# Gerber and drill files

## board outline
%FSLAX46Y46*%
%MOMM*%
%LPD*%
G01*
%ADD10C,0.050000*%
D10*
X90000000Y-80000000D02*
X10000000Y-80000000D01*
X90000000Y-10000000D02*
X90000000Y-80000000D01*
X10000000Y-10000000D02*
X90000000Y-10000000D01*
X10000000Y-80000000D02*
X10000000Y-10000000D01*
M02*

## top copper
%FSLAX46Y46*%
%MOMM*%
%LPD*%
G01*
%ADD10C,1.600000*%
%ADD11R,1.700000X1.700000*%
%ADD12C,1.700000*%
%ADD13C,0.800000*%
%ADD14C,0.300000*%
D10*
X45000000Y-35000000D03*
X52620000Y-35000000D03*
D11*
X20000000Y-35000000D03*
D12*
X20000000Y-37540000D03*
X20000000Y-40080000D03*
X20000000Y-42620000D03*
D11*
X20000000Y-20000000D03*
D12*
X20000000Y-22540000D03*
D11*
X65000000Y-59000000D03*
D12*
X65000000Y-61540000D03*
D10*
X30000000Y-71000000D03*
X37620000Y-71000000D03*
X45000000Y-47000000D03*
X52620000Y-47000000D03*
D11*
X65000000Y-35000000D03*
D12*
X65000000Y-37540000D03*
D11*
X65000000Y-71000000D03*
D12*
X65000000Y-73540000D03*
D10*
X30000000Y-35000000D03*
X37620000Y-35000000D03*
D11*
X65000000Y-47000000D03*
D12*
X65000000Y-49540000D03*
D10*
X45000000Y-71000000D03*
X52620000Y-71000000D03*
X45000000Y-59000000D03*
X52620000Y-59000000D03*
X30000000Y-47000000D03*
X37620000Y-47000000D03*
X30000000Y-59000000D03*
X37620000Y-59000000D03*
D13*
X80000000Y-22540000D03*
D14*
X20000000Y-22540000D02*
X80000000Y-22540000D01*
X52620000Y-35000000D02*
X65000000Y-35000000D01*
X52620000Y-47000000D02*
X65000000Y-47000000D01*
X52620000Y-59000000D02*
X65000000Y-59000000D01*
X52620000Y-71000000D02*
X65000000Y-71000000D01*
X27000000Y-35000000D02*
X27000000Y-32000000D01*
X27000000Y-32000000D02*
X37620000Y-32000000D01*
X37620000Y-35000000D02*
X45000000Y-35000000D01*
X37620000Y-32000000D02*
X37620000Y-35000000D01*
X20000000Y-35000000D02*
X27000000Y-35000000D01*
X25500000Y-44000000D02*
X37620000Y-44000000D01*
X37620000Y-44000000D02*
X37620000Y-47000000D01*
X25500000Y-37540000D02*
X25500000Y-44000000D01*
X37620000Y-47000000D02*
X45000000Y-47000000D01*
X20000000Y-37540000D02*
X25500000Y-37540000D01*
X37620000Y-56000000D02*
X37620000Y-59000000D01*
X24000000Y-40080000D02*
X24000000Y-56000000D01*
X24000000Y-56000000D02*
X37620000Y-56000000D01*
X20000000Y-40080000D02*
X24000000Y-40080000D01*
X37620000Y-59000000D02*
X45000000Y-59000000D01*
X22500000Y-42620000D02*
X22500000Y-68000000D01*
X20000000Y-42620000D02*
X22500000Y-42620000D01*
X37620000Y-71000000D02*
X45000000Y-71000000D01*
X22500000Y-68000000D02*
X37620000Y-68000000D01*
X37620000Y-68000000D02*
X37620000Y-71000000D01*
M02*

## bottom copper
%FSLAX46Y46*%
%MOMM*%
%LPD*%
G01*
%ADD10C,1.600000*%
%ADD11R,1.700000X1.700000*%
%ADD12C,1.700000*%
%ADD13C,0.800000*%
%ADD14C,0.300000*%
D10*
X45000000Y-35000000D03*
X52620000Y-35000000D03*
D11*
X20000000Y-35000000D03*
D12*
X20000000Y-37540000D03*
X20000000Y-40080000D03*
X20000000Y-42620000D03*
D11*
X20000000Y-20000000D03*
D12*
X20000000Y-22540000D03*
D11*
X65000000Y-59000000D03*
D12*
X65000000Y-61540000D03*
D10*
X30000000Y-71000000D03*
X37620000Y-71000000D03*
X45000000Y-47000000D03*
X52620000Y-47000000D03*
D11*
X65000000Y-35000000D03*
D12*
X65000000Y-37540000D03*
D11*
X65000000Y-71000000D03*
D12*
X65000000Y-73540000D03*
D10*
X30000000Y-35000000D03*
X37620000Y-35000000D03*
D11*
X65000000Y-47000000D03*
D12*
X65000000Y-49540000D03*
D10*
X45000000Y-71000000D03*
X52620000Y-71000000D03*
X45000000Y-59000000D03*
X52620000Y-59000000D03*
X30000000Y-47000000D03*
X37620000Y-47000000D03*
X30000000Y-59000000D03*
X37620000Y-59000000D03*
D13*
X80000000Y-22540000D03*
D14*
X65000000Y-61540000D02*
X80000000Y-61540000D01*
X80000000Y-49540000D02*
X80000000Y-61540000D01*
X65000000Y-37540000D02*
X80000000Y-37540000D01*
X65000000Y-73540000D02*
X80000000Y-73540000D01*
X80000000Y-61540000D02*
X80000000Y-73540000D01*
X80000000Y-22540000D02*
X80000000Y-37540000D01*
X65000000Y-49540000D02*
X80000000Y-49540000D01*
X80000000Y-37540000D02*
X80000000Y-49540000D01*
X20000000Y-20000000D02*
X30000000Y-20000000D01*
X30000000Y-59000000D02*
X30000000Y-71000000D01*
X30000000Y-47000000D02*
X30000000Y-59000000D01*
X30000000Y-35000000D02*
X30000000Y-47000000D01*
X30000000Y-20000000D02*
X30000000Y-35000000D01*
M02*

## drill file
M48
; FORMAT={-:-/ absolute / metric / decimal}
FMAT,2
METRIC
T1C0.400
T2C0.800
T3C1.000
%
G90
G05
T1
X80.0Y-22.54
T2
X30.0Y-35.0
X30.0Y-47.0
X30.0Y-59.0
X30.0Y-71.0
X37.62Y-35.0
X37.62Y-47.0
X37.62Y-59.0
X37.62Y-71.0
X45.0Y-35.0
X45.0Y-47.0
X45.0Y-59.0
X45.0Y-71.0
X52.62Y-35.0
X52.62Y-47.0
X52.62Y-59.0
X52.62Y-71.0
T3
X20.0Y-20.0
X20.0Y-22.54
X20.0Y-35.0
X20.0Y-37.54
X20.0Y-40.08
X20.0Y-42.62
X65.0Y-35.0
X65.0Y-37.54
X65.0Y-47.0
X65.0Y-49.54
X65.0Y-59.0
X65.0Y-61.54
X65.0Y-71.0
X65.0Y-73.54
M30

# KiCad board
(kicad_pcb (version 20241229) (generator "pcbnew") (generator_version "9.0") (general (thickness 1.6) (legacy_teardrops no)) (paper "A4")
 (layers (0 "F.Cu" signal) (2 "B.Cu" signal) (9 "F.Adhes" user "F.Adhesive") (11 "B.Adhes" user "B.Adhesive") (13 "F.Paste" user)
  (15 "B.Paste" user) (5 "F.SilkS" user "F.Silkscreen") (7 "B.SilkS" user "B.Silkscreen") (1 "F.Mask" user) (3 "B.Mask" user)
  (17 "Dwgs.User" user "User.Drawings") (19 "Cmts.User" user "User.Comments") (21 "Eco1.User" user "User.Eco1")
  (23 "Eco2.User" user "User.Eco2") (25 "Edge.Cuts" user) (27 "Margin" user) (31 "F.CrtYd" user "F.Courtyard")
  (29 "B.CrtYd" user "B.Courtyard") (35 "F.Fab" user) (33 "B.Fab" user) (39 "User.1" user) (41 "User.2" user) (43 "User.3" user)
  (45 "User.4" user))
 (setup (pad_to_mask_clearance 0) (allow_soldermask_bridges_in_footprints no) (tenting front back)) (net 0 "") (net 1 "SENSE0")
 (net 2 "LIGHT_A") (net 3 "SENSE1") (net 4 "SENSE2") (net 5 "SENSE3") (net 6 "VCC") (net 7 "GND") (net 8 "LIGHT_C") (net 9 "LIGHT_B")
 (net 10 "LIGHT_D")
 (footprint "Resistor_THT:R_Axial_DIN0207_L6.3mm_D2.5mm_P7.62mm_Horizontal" (layer "F.Cu") (at 45 35)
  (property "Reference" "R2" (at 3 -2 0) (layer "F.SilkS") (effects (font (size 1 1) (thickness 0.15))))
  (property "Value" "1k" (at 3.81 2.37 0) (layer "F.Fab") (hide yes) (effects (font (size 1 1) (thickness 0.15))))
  (pad "1" thru_hole circle (at 0 0) (size 1.6 1.6) (drill 0.8) (layers "*.Cu" "*.Mask") (remove_unused_layers no) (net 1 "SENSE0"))
  (pad "2" thru_hole circle (at 7.62 0) (size 1.6 1.6) (drill 0.8) (layers "*.Cu" "*.Mask") (remove_unused_layers no) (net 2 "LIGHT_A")))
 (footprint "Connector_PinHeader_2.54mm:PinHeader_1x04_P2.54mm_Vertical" (layer "F.Cu") (at 20 35)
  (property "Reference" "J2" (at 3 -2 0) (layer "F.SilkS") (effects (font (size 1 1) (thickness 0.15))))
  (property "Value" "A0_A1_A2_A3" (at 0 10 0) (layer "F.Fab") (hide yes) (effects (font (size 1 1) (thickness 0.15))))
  (pad "1" thru_hole rect (at 0 0) (size 1.7 1.7) (drill 1) (layers "*.Cu" "*.Mask") (remove_unused_layers no) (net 1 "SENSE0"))
  (pad "2" thru_hole circle (at 0 2.54) (size 1.7 1.7) (drill 1) (layers "*.Cu" "*.Mask") (remove_unused_layers no) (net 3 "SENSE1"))
  (pad "3" thru_hole circle (at 0 5.08) (size 1.7 1.7) (drill 1) (layers "*.Cu" "*.Mask") (remove_unused_layers no) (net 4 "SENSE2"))
  (pad "4" thru_hole circle (at 0 7.62) (size 1.7 1.7) (drill 1) (layers "*.Cu" "*.Mask") (remove_unused_layers no) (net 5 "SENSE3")))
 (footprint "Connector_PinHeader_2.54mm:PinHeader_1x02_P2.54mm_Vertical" (layer "F.Cu") (at 20 20)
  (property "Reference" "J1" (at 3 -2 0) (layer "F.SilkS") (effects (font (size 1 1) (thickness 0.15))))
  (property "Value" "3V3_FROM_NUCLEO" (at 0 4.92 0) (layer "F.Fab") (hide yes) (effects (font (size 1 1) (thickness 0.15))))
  (pad "1" thru_hole rect (at 0 0) (size 1.7 1.7) (drill 1) (layers "*.Cu" "*.Mask") (remove_unused_layers no) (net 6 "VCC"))
  (pad "2" thru_hole circle (at 0 2.54) (size 1.7 1.7) (drill 1) (layers "*.Cu" "*.Mask") (remove_unused_layers no) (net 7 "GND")))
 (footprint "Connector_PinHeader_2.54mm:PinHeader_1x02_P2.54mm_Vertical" (layer "F.Cu") (at 65 59)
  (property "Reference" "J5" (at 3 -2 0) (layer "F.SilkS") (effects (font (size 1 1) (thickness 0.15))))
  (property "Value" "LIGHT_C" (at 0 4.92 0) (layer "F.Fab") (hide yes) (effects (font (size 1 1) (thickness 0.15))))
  (pad "1" thru_hole rect (at 0 0) (size 1.7 1.7) (drill 1) (layers "*.Cu" "*.Mask") (remove_unused_layers no) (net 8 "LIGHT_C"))
  (pad "2" thru_hole circle (at 0 2.54) (size 1.7 1.7) (drill 1) (layers "*.Cu" "*.Mask") (remove_unused_layers no) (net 7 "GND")))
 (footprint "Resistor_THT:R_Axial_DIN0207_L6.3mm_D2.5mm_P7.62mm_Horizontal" (layer "F.Cu") (at 30 71)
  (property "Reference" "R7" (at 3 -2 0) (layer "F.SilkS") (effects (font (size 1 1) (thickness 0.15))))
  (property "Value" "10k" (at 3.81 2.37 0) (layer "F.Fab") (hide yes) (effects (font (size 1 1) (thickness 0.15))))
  (pad "1" thru_hole circle (at 0 0) (size 1.6 1.6) (drill 0.8) (layers "*.Cu" "*.Mask") (remove_unused_layers no) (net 6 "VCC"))
  (pad "2" thru_hole circle (at 7.62 0) (size 1.6 1.6) (drill 0.8) (layers "*.Cu" "*.Mask") (remove_unused_layers no) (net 5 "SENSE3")))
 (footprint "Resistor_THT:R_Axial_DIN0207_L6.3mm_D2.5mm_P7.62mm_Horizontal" (layer "F.Cu") (at 45 47)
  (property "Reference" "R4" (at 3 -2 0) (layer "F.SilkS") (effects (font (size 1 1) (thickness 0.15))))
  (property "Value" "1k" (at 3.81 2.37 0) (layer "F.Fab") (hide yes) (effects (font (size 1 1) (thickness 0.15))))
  (pad "1" thru_hole circle (at 0 0) (size 1.6 1.6) (drill 0.8) (layers "*.Cu" "*.Mask") (remove_unused_layers no) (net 3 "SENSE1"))
  (pad "2" thru_hole circle (at 7.62 0) (size 1.6 1.6) (drill 0.8) (layers "*.Cu" "*.Mask") (remove_unused_layers no) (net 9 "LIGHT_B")))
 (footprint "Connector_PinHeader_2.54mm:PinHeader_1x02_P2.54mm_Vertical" (layer "F.Cu") (at 65 35)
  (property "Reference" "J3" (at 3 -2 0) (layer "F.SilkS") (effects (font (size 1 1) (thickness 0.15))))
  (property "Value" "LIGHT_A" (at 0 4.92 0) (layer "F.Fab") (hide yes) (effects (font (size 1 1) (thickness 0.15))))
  (pad "1" thru_hole rect (at 0 0) (size 1.7 1.7) (drill 1) (layers "*.Cu" "*.Mask") (remove_unused_layers no) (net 2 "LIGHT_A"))
  (pad "2" thru_hole circle (at 0 2.54) (size 1.7 1.7) (drill 1) (layers "*.Cu" "*.Mask") (remove_unused_layers no) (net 7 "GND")))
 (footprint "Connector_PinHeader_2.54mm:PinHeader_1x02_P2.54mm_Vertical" (layer "F.Cu") (at 65 71)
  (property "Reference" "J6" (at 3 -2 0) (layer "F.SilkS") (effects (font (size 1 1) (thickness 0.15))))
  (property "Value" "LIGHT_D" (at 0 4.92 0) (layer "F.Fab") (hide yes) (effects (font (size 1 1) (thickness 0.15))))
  (pad "1" thru_hole rect (at 0 0) (size 1.7 1.7) (drill 1) (layers "*.Cu" "*.Mask") (remove_unused_layers no) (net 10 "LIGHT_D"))
  (pad "2" thru_hole circle (at 0 2.54) (size 1.7 1.7) (drill 1) (layers "*.Cu" "*.Mask") (remove_unused_layers no) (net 7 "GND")))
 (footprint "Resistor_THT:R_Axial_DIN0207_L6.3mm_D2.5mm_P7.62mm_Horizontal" (layer "F.Cu") (at 30 35)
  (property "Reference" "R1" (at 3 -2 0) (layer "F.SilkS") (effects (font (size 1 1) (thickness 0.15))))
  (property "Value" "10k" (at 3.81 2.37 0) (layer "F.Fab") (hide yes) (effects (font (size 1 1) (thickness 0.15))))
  (pad "1" thru_hole circle (at 0 0) (size 1.6 1.6) (drill 0.8) (layers "*.Cu" "*.Mask") (remove_unused_layers no) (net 6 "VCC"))
  (pad "2" thru_hole circle (at 7.62 0) (size 1.6 1.6) (drill 0.8) (layers "*.Cu" "*.Mask") (remove_unused_layers no) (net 1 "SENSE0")))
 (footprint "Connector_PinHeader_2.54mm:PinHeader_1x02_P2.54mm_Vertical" (layer "F.Cu") (at 65 47)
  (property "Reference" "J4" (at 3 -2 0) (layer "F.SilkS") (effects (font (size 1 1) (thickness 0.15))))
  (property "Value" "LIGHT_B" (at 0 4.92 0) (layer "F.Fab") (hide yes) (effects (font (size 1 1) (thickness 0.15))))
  (pad "1" thru_hole rect (at 0 0) (size 1.7 1.7) (drill 1) (layers "*.Cu" "*.Mask") (remove_unused_layers no) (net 9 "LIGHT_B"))
  (pad "2" thru_hole circle (at 0 2.54) (size 1.7 1.7) (drill 1) (layers "*.Cu" "*.Mask") (remove_unused_layers no) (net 7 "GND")))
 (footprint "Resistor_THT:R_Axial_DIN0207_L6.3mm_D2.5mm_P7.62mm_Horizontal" (layer "F.Cu") (at 45 71)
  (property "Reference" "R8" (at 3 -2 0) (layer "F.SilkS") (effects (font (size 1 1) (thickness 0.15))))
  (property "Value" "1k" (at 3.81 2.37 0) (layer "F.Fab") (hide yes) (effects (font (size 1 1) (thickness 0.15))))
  (pad "1" thru_hole circle (at 0 0) (size 1.6 1.6) (drill 0.8) (layers "*.Cu" "*.Mask") (remove_unused_layers no) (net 5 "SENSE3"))
  (pad "2" thru_hole circle (at 7.62 0) (size 1.6 1.6) (drill 0.8) (layers "*.Cu" "*.Mask") (remove_unused_layers no) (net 10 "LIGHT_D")))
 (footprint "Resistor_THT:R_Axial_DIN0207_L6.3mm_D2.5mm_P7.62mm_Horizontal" (layer "F.Cu") (at 45 59)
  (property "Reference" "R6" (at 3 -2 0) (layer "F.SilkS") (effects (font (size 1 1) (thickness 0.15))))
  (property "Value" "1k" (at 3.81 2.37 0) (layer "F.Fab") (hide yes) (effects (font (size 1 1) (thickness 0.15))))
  (pad "1" thru_hole circle (at 0 0) (size 1.6 1.6) (drill 0.8) (layers "*.Cu" "*.Mask") (remove_unused_layers no) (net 4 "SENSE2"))
  (pad "2" thru_hole circle (at 7.62 0) (size 1.6 1.6) (drill 0.8) (layers "*.Cu" "*.Mask") (remove_unused_layers no) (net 8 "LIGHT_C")))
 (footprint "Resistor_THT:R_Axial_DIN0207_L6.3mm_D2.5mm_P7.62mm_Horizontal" (layer "F.Cu") (at 30 47)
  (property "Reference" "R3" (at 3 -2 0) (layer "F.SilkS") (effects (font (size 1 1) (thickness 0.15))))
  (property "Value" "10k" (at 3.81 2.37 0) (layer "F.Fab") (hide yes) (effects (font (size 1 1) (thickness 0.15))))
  (pad "1" thru_hole circle (at 0 0) (size 1.6 1.6) (drill 0.8) (layers "*.Cu" "*.Mask") (remove_unused_layers no) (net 6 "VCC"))
  (pad "2" thru_hole circle (at 7.62 0) (size 1.6 1.6) (drill 0.8) (layers "*.Cu" "*.Mask") (remove_unused_layers no) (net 3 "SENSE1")))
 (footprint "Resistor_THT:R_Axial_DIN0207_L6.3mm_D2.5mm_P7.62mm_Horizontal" (layer "F.Cu") (at 30 59)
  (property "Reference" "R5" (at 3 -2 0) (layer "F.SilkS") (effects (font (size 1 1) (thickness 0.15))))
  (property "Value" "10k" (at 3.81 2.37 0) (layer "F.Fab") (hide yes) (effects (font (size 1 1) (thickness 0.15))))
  (pad "1" thru_hole circle (at 0 0) (size 1.6 1.6) (drill 0.8) (layers "*.Cu" "*.Mask") (remove_unused_layers no) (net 6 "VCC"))
  (pad "2" thru_hole circle (at 7.62 0) (size 1.6 1.6) (drill 0.8) (layers "*.Cu" "*.Mask") (remove_unused_layers no) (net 4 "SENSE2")))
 (gr_line (start 90 80) (end 10 80) (stroke (width 0.05) (type default)) (layer "Edge.Cuts"))
 (gr_line (start 90 10) (end 90 80) (stroke (width 0.05) (type default)) (layer "Edge.Cuts"))
 (gr_line (start 10 10) (end 90 10) (stroke (width 0.05) (type default)) (layer "Edge.Cuts"))
 (gr_line (start 10 80) (end 10 10) (stroke (width 0.05) (type default)) (layer "Edge.Cuts"))
 (segment (start 20 22.54) (end 80 22.54) (width 0.3) (layer "F.Cu") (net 7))
 (via (at 80 22.54) (size 0.8) (drill 0.4) (layers "F.Cu" "B.Cu") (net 7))
 (segment (start 65 61.54) (end 80 61.54) (width 0.3) (layer "B.Cu") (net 7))
 (segment (start 80 49.54) (end 80 61.54) (width 0.3) (layer "B.Cu") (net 7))
 (segment (start 65 37.54) (end 80 37.54) (width 0.3) (layer "B.Cu") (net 7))
 (segment (start 65 73.54) (end 80 73.54) (width 0.3) (layer "B.Cu") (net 7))
 (segment (start 80 61.54) (end 80 73.54) (width 0.3) (layer "B.Cu") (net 7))
 (segment (start 80 22.54) (end 80 37.54) (width 0.3) (layer "B.Cu") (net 7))
 (segment (start 65 49.54) (end 80 49.54) (width 0.3) (layer "B.Cu") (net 7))
 (segment (start 80 37.54) (end 80 49.54) (width 0.3) (layer "B.Cu") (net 7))
 (segment (start 52.62 35) (end 65 35) (width 0.3) (layer "F.Cu") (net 2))
 (segment (start 52.62 47) (end 65 47) (width 0.3) (layer "F.Cu") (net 9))
 (segment (start 52.62 59) (end 65 59) (width 0.3) (layer "F.Cu") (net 8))
 (segment (start 52.62 71) (end 65 71) (width 0.3) (layer "F.Cu") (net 10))
 (segment (start 27 35) (end 27 32) (width 0.3) (layer "F.Cu") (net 1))
 (segment (start 27 32) (end 37.62 32) (width 0.3) (layer "F.Cu") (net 1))
 (segment (start 37.62 35) (end 45 35) (width 0.3) (layer "F.Cu") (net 1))
 (segment (start 37.62 32) (end 37.62 35) (width 0.3) (layer "F.Cu") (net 1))
 (segment (start 20 35) (end 27 35) (width 0.3) (layer "F.Cu") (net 1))
 (segment (start 25.5 44) (end 37.62 44) (width 0.3) (layer "F.Cu") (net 3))
 (segment (start 37.62 44) (end 37.62 47) (width 0.3) (layer "F.Cu") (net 3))
 (segment (start 25.5 37.54) (end 25.5 44) (width 0.3) (layer "F.Cu") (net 3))
 (segment (start 37.62 47) (end 45 47) (width 0.3) (layer "F.Cu") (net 3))
 (segment (start 20 37.54) (end 25.5 37.54) (width 0.3) (layer "F.Cu") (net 3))
 (segment (start 37.62 56) (end 37.62 59) (width 0.3) (layer "F.Cu") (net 4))
 (segment (start 24 40.08) (end 24 56) (width 0.3) (layer "F.Cu") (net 4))
 (segment (start 24 56) (end 37.62 56) (width 0.3) (layer "F.Cu") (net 4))
 (segment (start 20 40.08) (end 24 40.08) (width 0.3) (layer "F.Cu") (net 4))
 (segment (start 37.62 59) (end 45 59) (width 0.3) (layer "F.Cu") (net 4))
 (segment (start 22.5 42.62) (end 22.5 68) (width 0.3) (layer "F.Cu") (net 5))
 (segment (start 20 42.62) (end 22.5 42.62) (width 0.3) (layer "F.Cu") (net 5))
 (segment (start 37.62 71) (end 45 71) (width 0.3) (layer "F.Cu") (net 5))
 (segment (start 22.5 68) (end 37.62 68) (width 0.3) (layer "F.Cu") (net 5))
 (segment (start 37.62 68) (end 37.62 71) (width 0.3) (layer "F.Cu") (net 5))
 (segment (start 20 20) (end 30 20) (width 0.3) (layer "B.Cu") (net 6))
 (segment (start 30 59) (end 30 71) (width 0.3) (layer "B.Cu") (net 6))
 (segment (start 30 47) (end 30 59) (width 0.3) (layer "B.Cu") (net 6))
 (segment (start 30 35) (end 30 47) (width 0.3) (layer "B.Cu") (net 6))
 (segment (start 30 20) (end 30 35) (width 0.3) (layer "B.Cu") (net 6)))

